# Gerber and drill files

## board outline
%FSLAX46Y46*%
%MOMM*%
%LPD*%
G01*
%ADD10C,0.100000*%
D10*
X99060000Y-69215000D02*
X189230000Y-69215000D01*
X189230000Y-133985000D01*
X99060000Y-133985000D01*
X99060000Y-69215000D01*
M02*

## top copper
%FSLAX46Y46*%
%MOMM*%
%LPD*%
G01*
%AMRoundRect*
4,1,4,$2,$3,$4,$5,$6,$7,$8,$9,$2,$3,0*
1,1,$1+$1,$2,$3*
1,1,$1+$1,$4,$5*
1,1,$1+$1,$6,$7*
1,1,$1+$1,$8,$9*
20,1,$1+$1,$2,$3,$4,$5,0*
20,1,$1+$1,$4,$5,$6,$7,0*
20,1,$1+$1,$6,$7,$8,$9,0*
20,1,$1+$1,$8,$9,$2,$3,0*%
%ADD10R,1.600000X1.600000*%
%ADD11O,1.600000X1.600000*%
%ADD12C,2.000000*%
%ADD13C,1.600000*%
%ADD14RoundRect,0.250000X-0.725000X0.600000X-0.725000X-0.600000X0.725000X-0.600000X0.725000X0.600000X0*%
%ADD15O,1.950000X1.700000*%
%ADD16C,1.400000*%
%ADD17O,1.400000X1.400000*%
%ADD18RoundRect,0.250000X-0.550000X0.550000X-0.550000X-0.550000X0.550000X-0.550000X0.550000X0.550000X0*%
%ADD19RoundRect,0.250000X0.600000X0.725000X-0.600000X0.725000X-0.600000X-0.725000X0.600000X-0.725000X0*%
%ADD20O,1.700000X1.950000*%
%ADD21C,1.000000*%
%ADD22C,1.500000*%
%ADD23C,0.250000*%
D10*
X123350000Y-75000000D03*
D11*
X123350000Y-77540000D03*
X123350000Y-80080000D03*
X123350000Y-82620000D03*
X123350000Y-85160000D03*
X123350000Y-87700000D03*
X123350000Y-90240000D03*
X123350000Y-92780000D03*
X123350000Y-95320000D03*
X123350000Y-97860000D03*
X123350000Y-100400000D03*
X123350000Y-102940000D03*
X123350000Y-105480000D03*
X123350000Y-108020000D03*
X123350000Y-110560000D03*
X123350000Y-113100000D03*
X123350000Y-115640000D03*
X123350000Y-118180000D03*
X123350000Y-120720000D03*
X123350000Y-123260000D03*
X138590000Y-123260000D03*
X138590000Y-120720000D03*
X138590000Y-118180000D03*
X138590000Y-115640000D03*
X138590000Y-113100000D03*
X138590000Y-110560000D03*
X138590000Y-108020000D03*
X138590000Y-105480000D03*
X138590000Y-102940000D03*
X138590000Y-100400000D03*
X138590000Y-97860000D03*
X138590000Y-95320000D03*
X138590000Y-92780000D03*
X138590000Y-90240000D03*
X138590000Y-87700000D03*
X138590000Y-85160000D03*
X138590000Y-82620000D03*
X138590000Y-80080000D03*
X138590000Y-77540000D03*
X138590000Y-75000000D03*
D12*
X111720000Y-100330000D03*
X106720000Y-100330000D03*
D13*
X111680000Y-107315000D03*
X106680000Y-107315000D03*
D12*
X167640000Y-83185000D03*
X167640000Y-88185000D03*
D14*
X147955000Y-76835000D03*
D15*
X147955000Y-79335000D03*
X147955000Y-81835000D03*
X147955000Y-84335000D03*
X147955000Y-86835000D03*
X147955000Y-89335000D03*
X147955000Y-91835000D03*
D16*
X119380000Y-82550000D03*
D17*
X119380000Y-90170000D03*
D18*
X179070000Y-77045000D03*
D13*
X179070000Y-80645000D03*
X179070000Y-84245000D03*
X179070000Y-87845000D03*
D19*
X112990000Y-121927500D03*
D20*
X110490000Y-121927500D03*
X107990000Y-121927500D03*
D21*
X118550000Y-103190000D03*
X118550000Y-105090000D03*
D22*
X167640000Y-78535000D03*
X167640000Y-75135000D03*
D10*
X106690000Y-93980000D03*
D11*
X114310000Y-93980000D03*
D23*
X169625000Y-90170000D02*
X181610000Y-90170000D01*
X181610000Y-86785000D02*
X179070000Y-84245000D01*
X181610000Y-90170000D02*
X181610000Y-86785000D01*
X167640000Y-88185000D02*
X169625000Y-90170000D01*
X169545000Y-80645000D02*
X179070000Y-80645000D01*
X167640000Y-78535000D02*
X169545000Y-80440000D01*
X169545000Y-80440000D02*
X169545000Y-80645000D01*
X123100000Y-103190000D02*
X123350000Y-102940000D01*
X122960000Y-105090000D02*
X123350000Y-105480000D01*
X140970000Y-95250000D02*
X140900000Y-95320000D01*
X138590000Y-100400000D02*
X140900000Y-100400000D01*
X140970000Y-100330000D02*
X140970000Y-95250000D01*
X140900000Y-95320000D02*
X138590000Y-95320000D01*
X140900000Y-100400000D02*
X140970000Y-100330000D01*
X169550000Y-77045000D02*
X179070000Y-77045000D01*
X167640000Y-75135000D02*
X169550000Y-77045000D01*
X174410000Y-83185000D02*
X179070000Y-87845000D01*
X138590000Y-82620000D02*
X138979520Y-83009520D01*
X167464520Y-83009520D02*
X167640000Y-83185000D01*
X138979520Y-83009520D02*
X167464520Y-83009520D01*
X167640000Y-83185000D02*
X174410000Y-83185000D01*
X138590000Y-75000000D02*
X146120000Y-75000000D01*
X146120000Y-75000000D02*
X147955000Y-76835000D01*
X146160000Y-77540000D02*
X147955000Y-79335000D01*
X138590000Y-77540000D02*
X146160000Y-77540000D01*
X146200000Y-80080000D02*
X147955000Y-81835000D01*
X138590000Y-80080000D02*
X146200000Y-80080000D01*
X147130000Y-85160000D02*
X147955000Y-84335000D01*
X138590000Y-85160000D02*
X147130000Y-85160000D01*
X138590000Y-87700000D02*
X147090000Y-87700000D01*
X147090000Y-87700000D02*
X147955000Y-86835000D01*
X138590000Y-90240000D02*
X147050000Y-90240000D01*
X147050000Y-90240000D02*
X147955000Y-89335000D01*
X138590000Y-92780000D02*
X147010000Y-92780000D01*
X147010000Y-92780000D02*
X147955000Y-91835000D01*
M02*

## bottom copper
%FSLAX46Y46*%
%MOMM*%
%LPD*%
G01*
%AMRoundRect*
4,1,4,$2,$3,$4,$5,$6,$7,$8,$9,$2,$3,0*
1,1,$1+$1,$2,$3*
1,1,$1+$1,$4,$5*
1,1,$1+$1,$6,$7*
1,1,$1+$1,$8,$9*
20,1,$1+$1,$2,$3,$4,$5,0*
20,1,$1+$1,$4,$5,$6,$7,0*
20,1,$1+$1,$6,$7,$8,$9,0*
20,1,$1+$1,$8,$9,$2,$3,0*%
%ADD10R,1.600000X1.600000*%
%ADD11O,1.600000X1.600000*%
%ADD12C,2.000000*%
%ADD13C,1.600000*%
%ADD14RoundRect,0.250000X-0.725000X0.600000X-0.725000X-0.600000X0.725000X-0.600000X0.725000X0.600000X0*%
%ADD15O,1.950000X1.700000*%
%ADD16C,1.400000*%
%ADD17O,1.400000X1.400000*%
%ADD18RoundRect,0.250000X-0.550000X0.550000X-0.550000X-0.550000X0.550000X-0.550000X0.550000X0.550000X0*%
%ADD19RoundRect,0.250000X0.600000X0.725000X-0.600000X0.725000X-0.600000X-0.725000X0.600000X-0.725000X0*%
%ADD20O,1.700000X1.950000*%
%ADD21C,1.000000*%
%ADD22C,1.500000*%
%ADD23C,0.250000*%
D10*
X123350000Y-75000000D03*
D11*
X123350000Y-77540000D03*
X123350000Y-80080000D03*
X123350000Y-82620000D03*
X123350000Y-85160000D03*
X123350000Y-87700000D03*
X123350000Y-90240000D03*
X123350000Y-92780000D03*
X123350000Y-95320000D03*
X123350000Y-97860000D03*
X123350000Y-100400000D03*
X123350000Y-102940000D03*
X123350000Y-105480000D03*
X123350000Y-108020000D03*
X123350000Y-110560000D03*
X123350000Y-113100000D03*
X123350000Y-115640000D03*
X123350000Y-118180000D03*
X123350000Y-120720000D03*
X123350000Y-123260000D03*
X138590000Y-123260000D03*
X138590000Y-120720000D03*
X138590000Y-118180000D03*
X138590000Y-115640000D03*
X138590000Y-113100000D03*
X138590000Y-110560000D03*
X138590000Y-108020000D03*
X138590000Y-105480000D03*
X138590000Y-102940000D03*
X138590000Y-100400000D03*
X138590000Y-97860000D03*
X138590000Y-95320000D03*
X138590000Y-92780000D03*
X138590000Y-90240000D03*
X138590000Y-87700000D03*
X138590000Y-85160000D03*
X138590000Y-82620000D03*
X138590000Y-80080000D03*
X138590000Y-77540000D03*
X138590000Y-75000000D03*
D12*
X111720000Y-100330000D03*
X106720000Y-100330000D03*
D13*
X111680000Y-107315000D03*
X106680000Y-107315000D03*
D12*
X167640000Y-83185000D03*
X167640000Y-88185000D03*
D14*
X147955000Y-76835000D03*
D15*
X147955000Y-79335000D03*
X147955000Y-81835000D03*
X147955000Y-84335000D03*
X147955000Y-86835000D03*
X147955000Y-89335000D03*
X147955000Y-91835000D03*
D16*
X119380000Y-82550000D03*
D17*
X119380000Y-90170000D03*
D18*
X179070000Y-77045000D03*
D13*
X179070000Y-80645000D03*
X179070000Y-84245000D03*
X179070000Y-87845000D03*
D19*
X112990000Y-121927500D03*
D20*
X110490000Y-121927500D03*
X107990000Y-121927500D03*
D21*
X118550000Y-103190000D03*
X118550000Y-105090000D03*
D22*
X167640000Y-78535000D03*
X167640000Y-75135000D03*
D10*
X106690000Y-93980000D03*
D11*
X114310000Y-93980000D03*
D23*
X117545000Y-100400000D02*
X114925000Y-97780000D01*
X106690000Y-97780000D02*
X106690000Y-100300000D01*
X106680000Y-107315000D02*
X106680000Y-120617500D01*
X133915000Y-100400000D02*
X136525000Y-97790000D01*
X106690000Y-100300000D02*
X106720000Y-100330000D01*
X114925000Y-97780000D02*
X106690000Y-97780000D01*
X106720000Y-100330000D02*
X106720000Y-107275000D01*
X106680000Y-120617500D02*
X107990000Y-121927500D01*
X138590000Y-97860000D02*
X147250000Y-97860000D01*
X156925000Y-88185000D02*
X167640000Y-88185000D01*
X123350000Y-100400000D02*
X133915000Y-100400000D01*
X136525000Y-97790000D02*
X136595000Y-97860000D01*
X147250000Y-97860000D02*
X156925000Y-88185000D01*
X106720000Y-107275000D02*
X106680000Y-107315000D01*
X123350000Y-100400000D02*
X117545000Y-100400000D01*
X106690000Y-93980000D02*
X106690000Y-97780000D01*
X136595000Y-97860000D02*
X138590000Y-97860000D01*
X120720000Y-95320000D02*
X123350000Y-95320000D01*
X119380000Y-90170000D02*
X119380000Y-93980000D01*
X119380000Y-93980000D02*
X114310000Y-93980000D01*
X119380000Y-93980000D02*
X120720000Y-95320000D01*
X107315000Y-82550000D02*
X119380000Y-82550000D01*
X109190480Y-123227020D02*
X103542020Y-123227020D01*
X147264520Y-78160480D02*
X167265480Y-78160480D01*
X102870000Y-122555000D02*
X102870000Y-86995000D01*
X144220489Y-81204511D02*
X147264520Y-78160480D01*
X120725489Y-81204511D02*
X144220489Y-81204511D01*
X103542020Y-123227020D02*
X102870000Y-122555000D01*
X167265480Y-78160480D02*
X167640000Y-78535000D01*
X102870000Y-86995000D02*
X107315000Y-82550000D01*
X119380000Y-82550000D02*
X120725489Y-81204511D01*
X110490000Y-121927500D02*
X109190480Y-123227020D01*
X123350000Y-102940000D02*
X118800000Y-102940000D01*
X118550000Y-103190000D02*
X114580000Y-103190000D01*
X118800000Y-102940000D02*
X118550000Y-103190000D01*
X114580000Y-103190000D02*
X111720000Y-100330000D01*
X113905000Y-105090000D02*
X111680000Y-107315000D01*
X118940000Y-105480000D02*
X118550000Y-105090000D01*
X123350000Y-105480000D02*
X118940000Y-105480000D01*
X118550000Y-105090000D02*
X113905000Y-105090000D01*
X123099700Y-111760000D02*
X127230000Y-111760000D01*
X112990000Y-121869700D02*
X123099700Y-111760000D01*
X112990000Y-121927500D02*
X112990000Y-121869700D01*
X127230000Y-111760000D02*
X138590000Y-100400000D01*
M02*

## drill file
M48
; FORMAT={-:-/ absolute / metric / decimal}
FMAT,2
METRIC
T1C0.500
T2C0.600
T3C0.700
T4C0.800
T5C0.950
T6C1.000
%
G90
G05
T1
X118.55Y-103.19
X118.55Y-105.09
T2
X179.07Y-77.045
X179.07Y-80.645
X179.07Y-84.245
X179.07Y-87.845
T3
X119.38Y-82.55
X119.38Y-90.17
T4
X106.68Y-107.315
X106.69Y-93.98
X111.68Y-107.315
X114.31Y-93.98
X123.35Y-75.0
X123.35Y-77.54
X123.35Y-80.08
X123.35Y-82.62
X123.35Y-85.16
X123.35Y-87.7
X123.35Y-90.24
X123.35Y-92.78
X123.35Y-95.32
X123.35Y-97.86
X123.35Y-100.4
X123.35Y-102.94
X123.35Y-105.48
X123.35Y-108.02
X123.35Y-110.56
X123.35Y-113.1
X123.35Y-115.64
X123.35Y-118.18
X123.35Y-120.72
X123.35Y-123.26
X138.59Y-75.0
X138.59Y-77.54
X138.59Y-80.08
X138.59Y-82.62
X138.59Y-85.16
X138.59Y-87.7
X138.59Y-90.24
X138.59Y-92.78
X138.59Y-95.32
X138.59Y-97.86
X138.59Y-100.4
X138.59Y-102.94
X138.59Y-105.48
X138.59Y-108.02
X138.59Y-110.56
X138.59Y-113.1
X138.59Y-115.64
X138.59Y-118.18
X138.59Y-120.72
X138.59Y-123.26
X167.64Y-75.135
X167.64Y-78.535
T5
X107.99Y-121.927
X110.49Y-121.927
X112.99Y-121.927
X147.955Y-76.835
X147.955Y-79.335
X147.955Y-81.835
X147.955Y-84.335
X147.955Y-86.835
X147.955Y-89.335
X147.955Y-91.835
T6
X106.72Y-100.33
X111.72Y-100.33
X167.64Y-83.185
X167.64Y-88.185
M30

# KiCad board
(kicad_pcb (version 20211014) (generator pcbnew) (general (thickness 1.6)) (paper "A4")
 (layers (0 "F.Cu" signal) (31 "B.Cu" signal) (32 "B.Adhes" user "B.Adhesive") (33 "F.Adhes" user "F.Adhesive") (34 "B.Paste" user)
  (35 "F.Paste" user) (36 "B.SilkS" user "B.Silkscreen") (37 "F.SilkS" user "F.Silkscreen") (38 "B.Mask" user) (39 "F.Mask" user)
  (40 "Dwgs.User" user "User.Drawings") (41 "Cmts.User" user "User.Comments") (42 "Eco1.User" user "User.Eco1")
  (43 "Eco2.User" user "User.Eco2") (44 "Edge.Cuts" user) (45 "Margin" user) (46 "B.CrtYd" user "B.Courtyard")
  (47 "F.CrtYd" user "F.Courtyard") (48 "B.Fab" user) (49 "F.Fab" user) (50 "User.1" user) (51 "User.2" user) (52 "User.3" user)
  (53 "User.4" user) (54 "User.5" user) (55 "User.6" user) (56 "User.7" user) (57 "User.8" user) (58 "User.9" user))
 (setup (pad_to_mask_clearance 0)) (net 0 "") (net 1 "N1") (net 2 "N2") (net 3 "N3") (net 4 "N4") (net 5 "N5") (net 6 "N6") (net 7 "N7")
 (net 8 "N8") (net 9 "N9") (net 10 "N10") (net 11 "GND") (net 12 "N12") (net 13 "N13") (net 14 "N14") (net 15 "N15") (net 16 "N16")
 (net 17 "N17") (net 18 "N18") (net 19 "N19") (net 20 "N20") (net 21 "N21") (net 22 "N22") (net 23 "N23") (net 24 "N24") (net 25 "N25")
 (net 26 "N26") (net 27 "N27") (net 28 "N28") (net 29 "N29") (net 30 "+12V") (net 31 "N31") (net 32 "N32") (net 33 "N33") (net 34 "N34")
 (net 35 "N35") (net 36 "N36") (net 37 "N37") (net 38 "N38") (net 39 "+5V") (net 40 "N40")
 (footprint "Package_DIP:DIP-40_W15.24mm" (layer "F.Cu") (at 123.35 75)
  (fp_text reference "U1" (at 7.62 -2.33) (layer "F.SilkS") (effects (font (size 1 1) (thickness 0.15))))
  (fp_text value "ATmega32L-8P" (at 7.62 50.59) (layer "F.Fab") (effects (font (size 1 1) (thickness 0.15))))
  (pad "1" thru_hole rect (at 0 0) (size 1.6 1.6) (drill 0.8) (layers *.Cu *.Mask) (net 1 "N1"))
  (pad "2" thru_hole oval (at 0 2.54) (size 1.6 1.6) (drill 0.8) (layers *.Cu *.Mask) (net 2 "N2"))
  (pad "3" thru_hole oval (at 0 5.08) (size 1.6 1.6) (drill 0.8) (layers *.Cu *.Mask) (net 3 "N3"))
  (pad "4" thru_hole oval (at 0 7.62) (size 1.6 1.6) (drill 0.8) (layers *.Cu *.Mask) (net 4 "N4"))
  (pad "5" thru_hole oval (at 0 10.16) (size 1.6 1.6) (drill 0.8) (layers *.Cu *.Mask) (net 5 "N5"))
  (pad "6" thru_hole oval (at 0 12.7) (size 1.6 1.6) (drill 0.8) (layers *.Cu *.Mask) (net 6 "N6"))
  (pad "7" thru_hole oval (at 0 15.24) (size 1.6 1.6) (drill 0.8) (layers *.Cu *.Mask) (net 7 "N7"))
  (pad "8" thru_hole oval (at 0 17.78) (size 1.6 1.6) (drill 0.8) (layers *.Cu *.Mask) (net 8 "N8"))
  (pad "9" thru_hole oval (at 0 20.32) (size 1.6 1.6) (drill 0.8) (layers *.Cu *.Mask) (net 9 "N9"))
  (pad "10" thru_hole oval (at 0 22.86) (size 1.6 1.6) (drill 0.8) (layers *.Cu *.Mask) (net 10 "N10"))
  (pad "11" thru_hole oval (at 0 25.4) (size 1.6 1.6) (drill 0.8) (layers *.Cu *.Mask) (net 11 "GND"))
  (pad "12" thru_hole oval (at 0 27.94) (size 1.6 1.6) (drill 0.8) (layers *.Cu *.Mask) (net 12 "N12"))
  (pad "13" thru_hole oval (at 0 30.48) (size 1.6 1.6) (drill 0.8) (layers *.Cu *.Mask) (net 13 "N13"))
  (pad "14" thru_hole oval (at 0 33.02) (size 1.6 1.6) (drill 0.8) (layers *.Cu *.Mask) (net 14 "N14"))
  (pad "15" thru_hole oval (at 0 35.56) (size 1.6 1.6) (drill 0.8) (layers *.Cu *.Mask) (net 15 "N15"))
  (pad "16" thru_hole oval (at 0 38.1) (size 1.6 1.6) (drill 0.8) (layers *.Cu *.Mask) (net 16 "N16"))
  (pad "17" thru_hole oval (at 0 40.64) (size 1.6 1.6) (drill 0.8) (layers *.Cu *.Mask) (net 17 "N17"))
  (pad "18" thru_hole oval (at 0 43.18) (size 1.6 1.6) (drill 0.8) (layers *.Cu *.Mask) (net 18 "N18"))
  (pad "19" thru_hole oval (at 0 45.72) (size 1.6 1.6) (drill 0.8) (layers *.Cu *.Mask) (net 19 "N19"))
  (pad "20" thru_hole oval (at 0 48.26) (size 1.6 1.6) (drill 0.8) (layers *.Cu *.Mask) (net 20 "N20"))
  (pad "21" thru_hole oval (at 15.24 48.26) (size 1.6 1.6) (drill 0.8) (layers *.Cu *.Mask) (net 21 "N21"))
  (pad "22" thru_hole oval (at 15.24 45.72) (size 1.6 1.6) (drill 0.8) (layers *.Cu *.Mask) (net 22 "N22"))
  (pad "23" thru_hole oval (at 15.24 43.18) (size 1.6 1.6) (drill 0.8) (layers *.Cu *.Mask) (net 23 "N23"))
  (pad "24" thru_hole oval (at 15.24 40.64) (size 1.6 1.6) (drill 0.8) (layers *.Cu *.Mask) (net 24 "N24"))
  (pad "25" thru_hole oval (at 15.24 38.1) (size 1.6 1.6) (drill 0.8) (layers *.Cu *.Mask) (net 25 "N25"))
  (pad "26" thru_hole oval (at 15.24 35.56) (size 1.6 1.6) (drill 0.8) (layers *.Cu *.Mask) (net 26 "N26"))
  (pad "27" thru_hole oval (at 15.24 33.02) (size 1.6 1.6) (drill 0.8) (layers *.Cu *.Mask) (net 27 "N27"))
  (pad "28" thru_hole oval (at 15.24 30.48) (size 1.6 1.6) (drill 0.8) (layers *.Cu *.Mask) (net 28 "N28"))
  (pad "29" thru_hole oval (at 15.24 27.94) (size 1.6 1.6) (drill 0.8) (layers *.Cu *.Mask) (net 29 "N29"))
  (pad "30" thru_hole oval (at 15.24 25.4) (size 1.6 1.6) (drill 0.8) (layers *.Cu *.Mask) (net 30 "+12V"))
  (pad "31" thru_hole oval (at 15.24 22.86) (size 1.6 1.6) (drill 0.8) (layers *.Cu *.Mask) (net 11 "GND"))
  (pad "32" thru_hole oval (at 15.24 20.32) (size 1.6 1.6) (drill 0.8) (layers *.Cu *.Mask) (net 30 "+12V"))
  (pad "33" thru_hole oval (at 15.24 17.78) (size 1.6 1.6) (drill 0.8) (layers *.Cu *.Mask) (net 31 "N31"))
  (pad "34" thru_hole oval (at 15.24 15.24) (size 1.6 1.6) (drill 0.8) (layers *.Cu *.Mask) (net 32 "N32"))
  (pad "35" thru_hole oval (at 15.24 12.7) (size 1.6 1.6) (drill 0.8) (layers *.Cu *.Mask) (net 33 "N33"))
  (pad "36" thru_hole oval (at 15.24 10.16) (size 1.6 1.6) (drill 0.8) (layers *.Cu *.Mask) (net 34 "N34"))
  (pad "37" thru_hole oval (at 15.24 7.62) (size 1.6 1.6) (drill 0.8) (layers *.Cu *.Mask) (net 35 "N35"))
  (pad "38" thru_hole oval (at 15.24 5.08) (size 1.6 1.6) (drill 0.8) (layers *.Cu *.Mask) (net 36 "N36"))
  (pad "39" thru_hole oval (at 15.24 2.54) (size 1.6 1.6) (drill 0.8) (layers *.Cu *.Mask) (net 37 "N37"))
  (pad "40" thru_hole oval (at 15.24 0) (size 1.6 1.6) (drill 0.8) (layers *.Cu *.Mask) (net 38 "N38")))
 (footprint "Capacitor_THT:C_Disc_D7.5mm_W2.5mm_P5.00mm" (layer "F.Cu") (at 111.72 100.33 180)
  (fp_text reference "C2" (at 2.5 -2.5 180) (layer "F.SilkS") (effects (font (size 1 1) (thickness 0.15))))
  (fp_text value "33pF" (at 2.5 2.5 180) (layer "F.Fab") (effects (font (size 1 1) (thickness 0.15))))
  (pad "1" thru_hole circle (at 0 0 180) (size 2 2) (drill 1) (layers *.Cu *.Mask) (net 12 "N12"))
  (pad "2" thru_hole circle (at 5 0 180) (size 2 2) (drill 1) (layers *.Cu *.Mask) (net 11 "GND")))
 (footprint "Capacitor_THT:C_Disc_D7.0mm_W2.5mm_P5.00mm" (layer "F.Cu") (at 111.68 107.315 180)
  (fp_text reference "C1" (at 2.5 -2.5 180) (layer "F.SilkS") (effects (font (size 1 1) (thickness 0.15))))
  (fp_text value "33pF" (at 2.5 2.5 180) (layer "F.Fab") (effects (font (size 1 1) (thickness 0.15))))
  (pad "1" thru_hole circle (at 0 0 180) (size 1.6 1.6) (drill 0.8) (layers *.Cu *.Mask) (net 13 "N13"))
  (pad "2" thru_hole circle (at 5 0 180) (size 1.6 1.6) (drill 0.8) (layers *.Cu *.Mask) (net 11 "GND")))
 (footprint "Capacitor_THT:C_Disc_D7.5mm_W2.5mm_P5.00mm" (layer "F.Cu") (at 167.64 83.185 -90)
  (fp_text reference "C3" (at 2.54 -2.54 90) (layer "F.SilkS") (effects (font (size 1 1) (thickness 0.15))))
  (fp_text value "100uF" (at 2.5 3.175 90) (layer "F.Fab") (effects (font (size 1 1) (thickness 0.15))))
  (pad "1" thru_hole circle (at 0 0 270) (size 2 2) (drill 1) (layers *.Cu *.Mask) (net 35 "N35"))
  (pad "2" thru_hole circle (at 5 0 270) (size 2 2) (drill 1) (layers *.Cu *.Mask) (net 11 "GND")))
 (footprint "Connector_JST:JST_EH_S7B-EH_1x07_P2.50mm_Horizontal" (layer "F.Cu") (at 147.955 76.835 -90)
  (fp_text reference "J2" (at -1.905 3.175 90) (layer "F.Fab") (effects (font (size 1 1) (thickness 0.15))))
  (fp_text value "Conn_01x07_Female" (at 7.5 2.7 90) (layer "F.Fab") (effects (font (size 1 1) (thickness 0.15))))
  (pad "1" thru_hole roundrect (at 0 0 270) (size 1.7 1.95) (drill 0.95) (layers *.Cu *.Mask) (roundrect_rratio 0.147059) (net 38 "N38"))
  (pad "2" thru_hole oval (at 2.5 0 270) (size 1.7 1.95) (drill 0.95) (layers *.Cu *.Mask) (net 37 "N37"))
  (pad "3" thru_hole oval (at 5 0 270) (size 1.7 1.95) (drill 0.95) (layers *.Cu *.Mask) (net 36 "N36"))
  (pad "4" thru_hole oval (at 7.5 0 270) (size 1.7 1.95) (drill 0.95) (layers *.Cu *.Mask) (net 34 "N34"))
  (pad "5" thru_hole oval (at 10 0 270) (size 1.7 1.95) (drill 0.95) (layers *.Cu *.Mask) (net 33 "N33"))
  (pad "6" thru_hole oval (at 12.5 0 270) (size 1.7 1.95) (drill 0.95) (layers *.Cu *.Mask) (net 32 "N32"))
  (pad "7" thru_hole oval (at 15 0 270) (size 1.7 1.95) (drill 0.95) (layers *.Cu *.Mask) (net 31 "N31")))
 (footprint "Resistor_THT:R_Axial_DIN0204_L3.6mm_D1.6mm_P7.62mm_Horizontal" (layer "F.Cu") (at 119.38 82.55 -90)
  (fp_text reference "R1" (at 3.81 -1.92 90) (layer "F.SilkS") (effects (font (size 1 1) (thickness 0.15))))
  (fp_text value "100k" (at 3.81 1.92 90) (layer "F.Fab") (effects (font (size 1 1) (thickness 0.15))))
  (pad "1" thru_hole circle (at 0 0 270) (size 1.4 1.4) (drill 0.7) (layers *.Cu *.Mask) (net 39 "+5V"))
  (pad "2" thru_hole oval (at 7.62 0 270) (size 1.4 1.4) (drill 0.7) (layers *.Cu *.Mask) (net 9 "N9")))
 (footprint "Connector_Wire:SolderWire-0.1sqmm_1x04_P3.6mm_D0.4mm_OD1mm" (layer "F.Cu") (at 179.07 77.045 -90)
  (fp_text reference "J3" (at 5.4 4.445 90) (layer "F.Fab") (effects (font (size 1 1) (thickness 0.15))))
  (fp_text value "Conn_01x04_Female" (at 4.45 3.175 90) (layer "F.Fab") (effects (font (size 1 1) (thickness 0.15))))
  (pad "1" thru_hole roundrect (at 0 0 270) (size 1.6 1.6) (drill 0.6) (layers *.Cu *.Mask) (roundrect_rratio 0.15625) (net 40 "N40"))
  (pad "2" thru_hole circle (at 3.6 0 270) (size 1.6 1.6) (drill 0.6) (layers *.Cu *.Mask) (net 39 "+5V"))
  (pad "3" thru_hole circle (at 7.2 0 270) (size 1.6 1.6) (drill 0.6) (layers *.Cu *.Mask) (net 11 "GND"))
  (pad "4" thru_hole circle (at 10.8 0 270) (size 1.6 1.6) (drill 0.6) (layers *.Cu *.Mask) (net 35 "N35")))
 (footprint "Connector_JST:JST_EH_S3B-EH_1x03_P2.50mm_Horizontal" (layer "F.Cu") (at 112.99 121.9275 180)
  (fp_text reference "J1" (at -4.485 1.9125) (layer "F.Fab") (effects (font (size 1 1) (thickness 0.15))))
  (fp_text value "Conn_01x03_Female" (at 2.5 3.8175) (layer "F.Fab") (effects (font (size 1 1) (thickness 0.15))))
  (pad "1" thru_hole roundrect (at 0 0 180) (size 1.7 1.95) (drill 0.95) (layers *.Cu *.Mask) (roundrect_rratio 0.147059) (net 30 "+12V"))
  (pad "2" thru_hole oval (at 2.5 0 180) (size 1.7 1.95) (drill 0.95) (layers *.Cu *.Mask) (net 39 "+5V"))
  (pad "3" thru_hole oval (at 5 0 180) (size 1.7 1.95) (drill 0.95) (layers *.Cu *.Mask) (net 11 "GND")))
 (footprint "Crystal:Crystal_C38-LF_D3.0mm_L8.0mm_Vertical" (layer "F.Cu") (at 118.55 103.19 -90)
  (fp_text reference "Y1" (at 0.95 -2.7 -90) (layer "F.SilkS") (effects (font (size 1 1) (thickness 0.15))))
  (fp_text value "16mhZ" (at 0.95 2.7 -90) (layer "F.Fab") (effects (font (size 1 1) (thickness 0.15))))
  (pad "1" thru_hole circle (at 0 0 270) (size 1 1) (drill 0.5) (layers *.Cu *.Mask) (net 12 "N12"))
  (pad "2" thru_hole circle (at 1.9 0 270) (size 1 1) (drill 0.5) (layers *.Cu *.Mask) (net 13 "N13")))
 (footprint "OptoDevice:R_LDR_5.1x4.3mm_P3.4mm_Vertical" (layer "F.Cu") (at 167.64 78.535 90)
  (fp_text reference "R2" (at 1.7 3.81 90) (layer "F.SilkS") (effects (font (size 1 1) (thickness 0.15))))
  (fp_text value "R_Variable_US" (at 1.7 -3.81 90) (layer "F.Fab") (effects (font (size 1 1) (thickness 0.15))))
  (pad "1" thru_hole circle (at 0 0 90) (size 1.5 1.5) (drill 0.8) (layers *.Cu *.Mask) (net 39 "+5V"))
  (pad "2" thru_hole circle (at 3.4 0 90) (size 1.5 1.5) (drill 0.8) (layers *.Cu *.Mask) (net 40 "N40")))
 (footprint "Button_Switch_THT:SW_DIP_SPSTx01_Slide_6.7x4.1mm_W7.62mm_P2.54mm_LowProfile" (layer "F.Cu") (at 106.69 93.98)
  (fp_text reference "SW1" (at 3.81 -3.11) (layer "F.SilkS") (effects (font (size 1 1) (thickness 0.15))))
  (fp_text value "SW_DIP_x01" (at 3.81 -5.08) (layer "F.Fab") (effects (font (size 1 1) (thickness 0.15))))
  (pad "1" thru_hole rect (at 0 0) (size 1.6 1.6) (drill 0.8) (layers *.Cu *.Mask) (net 11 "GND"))
  (pad "2" thru_hole oval (at 7.62 0) (size 1.6 1.6) (drill 0.8) (layers *.Cu *.Mask) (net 9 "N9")))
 (gr_rect (start 99.06 69.215) (end 189.23 133.985) (layer "Edge.Cuts") (width 0.1) (fill none))
 (segment (start 169.625 90.17) (end 181.61 90.17) (width 0.25) (layer "F.Cu") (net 11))
 (segment (start 181.61 86.785) (end 179.07 84.245) (width 0.25) (layer "F.Cu") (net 11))
 (segment (start 181.61 90.17) (end 181.61 86.785) (width 0.25) (layer "F.Cu") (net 11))
 (segment (start 167.64 88.185) (end 169.625 90.17) (width 0.25) (layer "F.Cu") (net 11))
 (segment (start 117.545 100.4) (end 114.925 97.78) (width 0.25) (layer "B.Cu") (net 11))
 (segment (start 106.69 97.78) (end 106.69 100.3) (width 0.25) (layer "B.Cu") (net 11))
 (segment (start 106.68 107.315) (end 106.68 120.6175) (width 0.25) (layer "B.Cu") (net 11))
 (segment (start 133.915 100.4) (end 136.525 97.79) (width 0.25) (layer "B.Cu") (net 11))
 (segment (start 106.69 100.3) (end 106.72 100.33) (width 0.25) (layer "B.Cu") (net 11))
 (segment (start 114.925 97.78) (end 106.69 97.78) (width 0.25) (layer "B.Cu") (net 11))
 (segment (start 106.72 100.33) (end 106.72 107.275) (width 0.25) (layer "B.Cu") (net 11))
 (segment (start 106.68 120.6175) (end 107.99 121.9275) (width 0.25) (layer "B.Cu") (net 11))
 (segment (start 138.59 97.86) (end 147.25 97.86) (width 0.25) (layer "B.Cu") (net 11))
 (segment (start 156.925 88.185) (end 167.64 88.185) (width 0.25) (layer "B.Cu") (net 11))
 (segment (start 123.35 100.4) (end 133.915 100.4) (width 0.25) (layer "B.Cu") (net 11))
 (segment (start 136.525 97.79) (end 136.595 97.86) (width 0.25) (layer "B.Cu") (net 11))
 (segment (start 147.25 97.86) (end 156.925 88.185) (width 0.25) (layer "B.Cu") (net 11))
 (segment (start 106.72 107.275) (end 106.68 107.315) (width 0.25) (layer "B.Cu") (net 11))
 (segment (start 123.35 100.4) (end 117.545 100.4) (width 0.25) (layer "B.Cu") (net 11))
 (segment (start 106.69 93.98) (end 106.69 97.78) (width 0.25) (layer "B.Cu") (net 11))
 (segment (start 136.595 97.86) (end 138.59 97.86) (width 0.25) (layer "B.Cu") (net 11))
 (segment (start 120.72 95.32) (end 123.35 95.32) (width 0.25) (layer "B.Cu") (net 9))
 (segment (start 119.38 90.17) (end 119.38 93.98) (width 0.25) (layer "B.Cu") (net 9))
 (segment (start 119.38 93.98) (end 114.31 93.98) (width 0.25) (layer "B.Cu") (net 9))
 (segment (start 119.38 93.98) (end 120.72 95.32) (width 0.25) (layer "B.Cu") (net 9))
 (segment (start 169.545 80.645) (end 179.07 80.645) (width 0.25) (layer "F.Cu") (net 39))
 (segment (start 167.64 78.535) (end 169.545 80.44) (width 0.25) (layer "F.Cu") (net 39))
 (segment (start 169.545 80.44) (end 169.545 80.645) (width 0.25) (layer "F.Cu") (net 39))
 (segment (start 107.315 82.55) (end 119.38 82.55) (width 0.25) (layer "B.Cu") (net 39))
 (segment (start 109.19048 123.22702) (end 103.54202 123.22702) (width 0.25) (layer "B.Cu") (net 39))
 (segment (start 147.26452 78.16048) (end 167.26548 78.16048) (width 0.25) (layer "B.Cu") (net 39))
 (segment (start 102.87 122.555) (end 102.87 86.995) (width 0.25) (layer "B.Cu") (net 39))
 (segment (start 144.220489 81.204511) (end 147.26452 78.16048) (width 0.25) (layer "B.Cu") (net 39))
 (segment (start 120.725489 81.204511) (end 144.220489 81.204511) (width 0.25) (layer "B.Cu") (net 39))
 (segment (start 103.54202 123.22702) (end 102.87 122.555) (width 0.25) (layer "B.Cu") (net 39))
 (segment (start 167.26548 78.16048) (end 167.64 78.535) (width 0.25) (layer "B.Cu") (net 39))
 (segment (start 102.87 86.995) (end 107.315 82.55) (width 0.25) (layer "B.Cu") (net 39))
 (segment (start 119.38 82.55) (end 120.725489 81.204511) (width 0.25) (layer "B.Cu") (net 39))
 (segment (start 110.49 121.9275) (end 109.19048 123.22702) (width 0.25) (layer "B.Cu") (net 39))
 (segment (start 123.1 103.19) (end 123.35 102.94) (width 0.25) (layer "F.Cu") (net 12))
 (segment (start 123.35 102.94) (end 118.8 102.94) (width 0.25) (layer "B.Cu") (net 12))
 (segment (start 118.55 103.19) (end 114.58 103.19) (width 0.25) (layer "B.Cu") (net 12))
 (segment (start 118.8 102.94) (end 118.55 103.19) (width 0.25) (layer "B.Cu") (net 12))
 (segment (start 114.58 103.19) (end 111.72 100.33) (width 0.25) (layer "B.Cu") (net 12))
 (segment (start 122.96 105.09) (end 123.35 105.48) (width 0.25) (layer "F.Cu") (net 13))
 (segment (start 113.905 105.09) (end 111.68 107.315) (width 0.25) (layer "B.Cu") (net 13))
 (segment (start 118.94 105.48) (end 118.55 105.09) (width 0.25) (layer "B.Cu") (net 13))
 (segment (start 123.35 105.48) (end 118.94 105.48) (width 0.25) (layer "B.Cu") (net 13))
 (segment (start 118.55 105.09) (end 113.905 105.09) (width 0.25) (layer "B.Cu") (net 13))
 (segment (start 140.97 95.25) (end 140.9 95.32) (width 0.25) (layer "F.Cu") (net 30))
 (segment (start 138.59 100.4) (end 140.9 100.4) (width 0.25) (layer "F.Cu") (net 30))
 (segment (start 140.97 100.33) (end 140.97 95.25) (width 0.25) (layer "F.Cu") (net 30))
 (segment (start 140.9 95.32) (end 138.59 95.32) (width 0.25) (layer "F.Cu") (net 30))
 (segment (start 140.9 100.4) (end 140.97 100.33) (width 0.25) (layer "F.Cu") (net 30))
 (segment (start 123.0997 111.76) (end 127.23 111.76) (width 0.25) (layer "B.Cu") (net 30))
 (segment (start 112.99 121.8697) (end 123.0997 111.76) (width 0.25) (layer "B.Cu") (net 30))
 (segment (start 112.99 121.9275) (end 112.99 121.8697) (width 0.25) (layer "B.Cu") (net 30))
 (segment (start 127.23 111.76) (end 138.59 100.4) (width 0.25) (layer "B.Cu") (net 30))
 (segment (start 169.55 77.045) (end 179.07 77.045) (width 0.25) (layer "F.Cu") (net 40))
 (segment (start 167.64 75.135) (end 169.55 77.045) (width 0.25) (layer "F.Cu") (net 40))
 (segment (start 174.41 83.185) (end 179.07 87.845) (width 0.25) (layer "F.Cu") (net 35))
 (segment (start 138.59 82.62) (end 138.97952 83.00952) (width 0.25) (layer "F.Cu") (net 35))
 (segment (start 167.46452 83.00952) (end 167.64 83.185) (width 0.25) (layer "F.Cu") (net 35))
 (segment (start 138.97952 83.00952) (end 167.46452 83.00952) (width 0.25) (layer "F.Cu") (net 35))
 (segment (start 167.64 83.185) (end 174.41 83.185) (width 0.25) (layer "F.Cu") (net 35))
 (segment (start 138.59 75) (end 146.12 75) (width 0.25) (layer "F.Cu") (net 38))
 (segment (start 146.12 75) (end 147.955 76.835) (width 0.25) (layer "F.Cu") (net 38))
 (segment (start 146.16 77.54) (end 147.955 79.335) (width 0.25) (layer "F.Cu") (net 37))
 (segment (start 138.59 77.54) (end 146.16 77.54) (width 0.25) (layer "F.Cu") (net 37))
 (segment (start 146.2 80.08) (end 147.955 81.835) (width 0.25) (layer "F.Cu") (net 36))
 (segment (start 138.59 80.08) (end 146.2 80.08) (width 0.25) (layer "F.Cu") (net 36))
 (segment (start 147.13 85.16) (end 147.955 84.335) (width 0.25) (layer "F.Cu") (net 34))
 (segment (start 138.59 85.16) (end 147.13 85.16) (width 0.25) (layer "F.Cu") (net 34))
 (segment (start 138.59 87.7) (end 147.09 87.7) (width 0.25) (layer "F.Cu") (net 33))
 (segment (start 147.09 87.7) (end 147.955 86.835) (width 0.25) (layer "F.Cu") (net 33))
 (segment (start 138.59 90.24) (end 147.05 90.24) (width 0.25) (layer "F.Cu") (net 32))
 (segment (start 147.05 90.24) (end 147.955 89.335) (width 0.25) (layer "F.Cu") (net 32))
 (segment (start 138.59 92.78) (end 147.01 92.78) (width 0.25) (layer "F.Cu") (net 31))
 (segment (start 147.01 92.78) (end 147.955 91.835) (width 0.25) (layer "F.Cu") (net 31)))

